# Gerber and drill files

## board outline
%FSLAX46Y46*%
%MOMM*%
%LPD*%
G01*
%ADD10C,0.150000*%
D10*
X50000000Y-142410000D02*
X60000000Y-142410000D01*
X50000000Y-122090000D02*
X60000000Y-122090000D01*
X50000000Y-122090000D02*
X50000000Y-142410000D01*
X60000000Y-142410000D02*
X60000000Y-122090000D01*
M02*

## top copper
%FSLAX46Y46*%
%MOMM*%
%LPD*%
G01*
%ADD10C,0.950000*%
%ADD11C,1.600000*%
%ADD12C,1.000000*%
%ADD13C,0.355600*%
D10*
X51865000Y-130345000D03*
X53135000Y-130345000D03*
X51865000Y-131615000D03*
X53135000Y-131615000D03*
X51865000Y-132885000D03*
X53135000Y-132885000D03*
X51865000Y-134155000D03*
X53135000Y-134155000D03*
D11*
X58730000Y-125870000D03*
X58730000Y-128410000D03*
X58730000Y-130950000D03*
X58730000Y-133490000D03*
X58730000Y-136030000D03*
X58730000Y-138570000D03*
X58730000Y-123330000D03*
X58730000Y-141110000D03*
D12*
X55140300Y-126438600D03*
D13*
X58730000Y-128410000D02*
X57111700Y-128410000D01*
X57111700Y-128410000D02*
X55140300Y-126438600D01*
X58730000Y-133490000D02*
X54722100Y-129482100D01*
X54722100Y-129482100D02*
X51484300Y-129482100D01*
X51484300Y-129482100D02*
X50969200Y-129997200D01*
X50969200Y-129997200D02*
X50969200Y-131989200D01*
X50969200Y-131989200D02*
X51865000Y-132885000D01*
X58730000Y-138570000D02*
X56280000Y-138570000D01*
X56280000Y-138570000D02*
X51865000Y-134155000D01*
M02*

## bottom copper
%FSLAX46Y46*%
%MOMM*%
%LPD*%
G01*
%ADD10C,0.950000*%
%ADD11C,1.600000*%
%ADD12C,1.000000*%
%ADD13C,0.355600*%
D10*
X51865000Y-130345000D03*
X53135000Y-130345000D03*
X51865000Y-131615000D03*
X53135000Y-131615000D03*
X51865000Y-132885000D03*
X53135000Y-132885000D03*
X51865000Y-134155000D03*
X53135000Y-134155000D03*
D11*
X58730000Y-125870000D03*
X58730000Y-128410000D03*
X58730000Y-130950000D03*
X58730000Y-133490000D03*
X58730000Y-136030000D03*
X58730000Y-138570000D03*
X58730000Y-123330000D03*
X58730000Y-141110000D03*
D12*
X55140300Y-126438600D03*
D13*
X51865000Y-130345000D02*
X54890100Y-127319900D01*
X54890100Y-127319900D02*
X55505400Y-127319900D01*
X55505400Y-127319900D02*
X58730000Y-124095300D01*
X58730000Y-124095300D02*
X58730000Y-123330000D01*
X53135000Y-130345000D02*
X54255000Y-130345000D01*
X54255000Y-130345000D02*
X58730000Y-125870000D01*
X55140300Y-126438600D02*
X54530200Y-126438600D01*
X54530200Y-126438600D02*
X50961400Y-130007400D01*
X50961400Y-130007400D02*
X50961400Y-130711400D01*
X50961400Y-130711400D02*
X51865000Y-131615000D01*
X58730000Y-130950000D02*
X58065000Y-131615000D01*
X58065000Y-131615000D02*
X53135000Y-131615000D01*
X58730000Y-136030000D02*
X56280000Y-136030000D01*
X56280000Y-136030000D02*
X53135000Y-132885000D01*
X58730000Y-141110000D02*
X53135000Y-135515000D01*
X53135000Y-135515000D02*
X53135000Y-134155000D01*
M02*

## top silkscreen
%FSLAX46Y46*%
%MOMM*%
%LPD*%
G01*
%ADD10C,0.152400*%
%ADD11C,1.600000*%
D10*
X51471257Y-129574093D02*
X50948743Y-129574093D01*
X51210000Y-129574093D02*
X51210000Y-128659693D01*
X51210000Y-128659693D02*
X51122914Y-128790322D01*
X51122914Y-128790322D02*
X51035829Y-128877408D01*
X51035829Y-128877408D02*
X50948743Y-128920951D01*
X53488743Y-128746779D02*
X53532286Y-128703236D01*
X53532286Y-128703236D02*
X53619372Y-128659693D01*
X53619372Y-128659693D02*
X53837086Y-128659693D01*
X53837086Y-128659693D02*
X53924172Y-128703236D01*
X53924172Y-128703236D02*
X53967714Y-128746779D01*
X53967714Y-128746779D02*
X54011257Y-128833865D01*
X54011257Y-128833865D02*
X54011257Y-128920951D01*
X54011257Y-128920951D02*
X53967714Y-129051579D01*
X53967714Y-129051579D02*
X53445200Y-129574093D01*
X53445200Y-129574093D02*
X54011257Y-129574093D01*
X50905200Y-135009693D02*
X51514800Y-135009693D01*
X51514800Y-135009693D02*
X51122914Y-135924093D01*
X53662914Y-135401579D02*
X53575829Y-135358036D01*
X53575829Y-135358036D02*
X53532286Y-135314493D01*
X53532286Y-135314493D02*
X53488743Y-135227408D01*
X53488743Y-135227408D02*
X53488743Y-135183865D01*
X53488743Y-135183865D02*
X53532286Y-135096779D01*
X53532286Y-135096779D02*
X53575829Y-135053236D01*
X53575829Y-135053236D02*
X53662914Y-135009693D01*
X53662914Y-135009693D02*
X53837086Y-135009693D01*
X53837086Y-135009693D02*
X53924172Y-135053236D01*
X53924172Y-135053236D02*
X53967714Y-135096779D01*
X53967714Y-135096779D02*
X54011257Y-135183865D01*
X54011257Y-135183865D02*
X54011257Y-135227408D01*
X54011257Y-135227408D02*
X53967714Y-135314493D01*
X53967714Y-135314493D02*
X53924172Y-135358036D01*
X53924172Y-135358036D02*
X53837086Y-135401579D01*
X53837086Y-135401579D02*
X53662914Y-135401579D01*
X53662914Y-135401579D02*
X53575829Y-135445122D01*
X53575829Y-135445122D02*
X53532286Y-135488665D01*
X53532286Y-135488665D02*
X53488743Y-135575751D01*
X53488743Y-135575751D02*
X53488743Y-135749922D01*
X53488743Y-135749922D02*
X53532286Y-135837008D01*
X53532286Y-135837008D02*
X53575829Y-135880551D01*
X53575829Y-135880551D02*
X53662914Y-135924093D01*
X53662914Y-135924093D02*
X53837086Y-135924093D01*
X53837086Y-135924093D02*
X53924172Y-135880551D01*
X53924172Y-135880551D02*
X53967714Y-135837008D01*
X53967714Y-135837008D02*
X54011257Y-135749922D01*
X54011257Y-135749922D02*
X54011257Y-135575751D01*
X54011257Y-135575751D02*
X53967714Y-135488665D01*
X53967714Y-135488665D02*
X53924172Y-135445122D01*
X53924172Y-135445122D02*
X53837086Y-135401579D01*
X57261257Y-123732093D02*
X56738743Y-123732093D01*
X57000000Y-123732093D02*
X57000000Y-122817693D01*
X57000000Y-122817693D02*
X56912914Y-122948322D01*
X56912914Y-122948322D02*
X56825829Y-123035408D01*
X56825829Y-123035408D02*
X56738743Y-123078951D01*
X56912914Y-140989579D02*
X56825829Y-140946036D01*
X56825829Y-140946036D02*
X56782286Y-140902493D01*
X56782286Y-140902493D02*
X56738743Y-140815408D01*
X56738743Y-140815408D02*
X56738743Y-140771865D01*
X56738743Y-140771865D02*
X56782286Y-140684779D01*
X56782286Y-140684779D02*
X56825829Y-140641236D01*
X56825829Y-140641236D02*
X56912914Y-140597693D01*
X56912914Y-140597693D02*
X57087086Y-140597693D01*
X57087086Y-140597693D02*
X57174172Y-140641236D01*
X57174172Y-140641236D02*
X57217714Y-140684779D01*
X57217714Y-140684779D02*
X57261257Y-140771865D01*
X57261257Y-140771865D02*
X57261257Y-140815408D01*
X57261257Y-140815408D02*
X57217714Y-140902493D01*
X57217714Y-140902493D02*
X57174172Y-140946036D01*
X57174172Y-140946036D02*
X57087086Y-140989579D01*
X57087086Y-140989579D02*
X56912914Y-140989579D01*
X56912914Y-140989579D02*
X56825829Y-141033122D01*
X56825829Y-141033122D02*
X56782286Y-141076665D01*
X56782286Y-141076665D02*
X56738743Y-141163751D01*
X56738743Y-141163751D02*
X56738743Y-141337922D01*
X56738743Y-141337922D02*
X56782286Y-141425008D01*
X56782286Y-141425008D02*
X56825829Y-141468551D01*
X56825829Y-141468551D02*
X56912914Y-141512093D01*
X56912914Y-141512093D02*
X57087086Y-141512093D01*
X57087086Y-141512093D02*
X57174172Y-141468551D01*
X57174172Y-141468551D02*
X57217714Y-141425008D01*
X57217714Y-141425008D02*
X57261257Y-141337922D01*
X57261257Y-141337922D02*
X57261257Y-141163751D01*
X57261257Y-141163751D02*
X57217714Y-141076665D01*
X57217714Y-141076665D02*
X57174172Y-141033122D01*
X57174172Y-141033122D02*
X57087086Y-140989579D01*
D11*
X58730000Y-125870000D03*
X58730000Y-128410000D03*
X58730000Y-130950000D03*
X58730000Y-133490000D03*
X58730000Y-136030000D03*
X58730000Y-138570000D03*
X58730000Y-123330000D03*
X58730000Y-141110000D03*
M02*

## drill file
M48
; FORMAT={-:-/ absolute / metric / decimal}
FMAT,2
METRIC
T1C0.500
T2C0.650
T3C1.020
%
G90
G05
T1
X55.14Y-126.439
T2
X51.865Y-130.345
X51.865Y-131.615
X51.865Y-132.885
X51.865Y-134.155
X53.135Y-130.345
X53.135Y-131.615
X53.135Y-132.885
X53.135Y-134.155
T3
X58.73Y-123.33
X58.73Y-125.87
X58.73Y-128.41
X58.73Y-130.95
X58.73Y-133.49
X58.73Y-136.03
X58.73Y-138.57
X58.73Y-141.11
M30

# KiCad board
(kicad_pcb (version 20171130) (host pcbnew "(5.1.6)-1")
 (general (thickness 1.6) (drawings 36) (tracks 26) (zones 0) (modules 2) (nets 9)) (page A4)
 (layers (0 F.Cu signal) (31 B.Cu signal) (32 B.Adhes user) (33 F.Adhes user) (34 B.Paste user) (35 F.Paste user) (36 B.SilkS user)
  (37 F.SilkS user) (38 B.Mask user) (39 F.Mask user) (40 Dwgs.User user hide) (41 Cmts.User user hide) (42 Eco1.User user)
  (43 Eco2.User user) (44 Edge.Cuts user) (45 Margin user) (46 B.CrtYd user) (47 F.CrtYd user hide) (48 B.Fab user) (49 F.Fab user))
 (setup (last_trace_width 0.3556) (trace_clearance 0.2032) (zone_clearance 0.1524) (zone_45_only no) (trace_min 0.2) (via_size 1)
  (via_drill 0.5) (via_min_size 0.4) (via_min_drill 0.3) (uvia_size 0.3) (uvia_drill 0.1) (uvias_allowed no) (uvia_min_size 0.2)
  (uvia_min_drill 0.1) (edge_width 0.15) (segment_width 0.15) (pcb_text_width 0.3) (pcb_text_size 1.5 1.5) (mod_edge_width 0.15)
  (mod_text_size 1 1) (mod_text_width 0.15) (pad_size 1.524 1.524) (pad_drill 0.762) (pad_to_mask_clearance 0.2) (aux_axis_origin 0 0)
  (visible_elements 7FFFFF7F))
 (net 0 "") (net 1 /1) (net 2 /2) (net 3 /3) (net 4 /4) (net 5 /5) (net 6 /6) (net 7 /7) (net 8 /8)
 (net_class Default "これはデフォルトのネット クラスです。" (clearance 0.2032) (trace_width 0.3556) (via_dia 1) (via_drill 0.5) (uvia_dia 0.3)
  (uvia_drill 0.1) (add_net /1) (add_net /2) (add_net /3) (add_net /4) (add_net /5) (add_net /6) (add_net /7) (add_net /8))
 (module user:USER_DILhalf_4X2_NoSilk (layer F.Cu) (at 52.5 132.25)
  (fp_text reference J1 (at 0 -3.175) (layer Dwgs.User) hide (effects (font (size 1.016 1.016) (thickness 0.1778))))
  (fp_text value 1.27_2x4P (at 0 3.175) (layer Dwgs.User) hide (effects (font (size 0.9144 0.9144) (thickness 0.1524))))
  (pad 1 thru_hole circle (at -0.635 -1.905) (size 0.95 0.95) (drill 0.65) (layers *.Cu *.Mask) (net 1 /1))
  (pad 2 thru_hole circle (at 0.635 -1.905) (size 0.95 0.95) (drill 0.65) (layers *.Cu *.Mask) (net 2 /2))
  (pad 3 thru_hole circle (at -0.635 -0.635) (size 0.95 0.95) (drill 0.65) (layers *.Cu *.Mask) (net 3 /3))
  (pad 4 thru_hole circle (at 0.635 -0.635) (size 0.95 0.95) (drill 0.65) (layers *.Cu *.Mask) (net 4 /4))
  (pad 5 thru_hole circle (at -0.635 0.635) (size 0.95 0.95) (drill 0.65) (layers *.Cu *.Mask) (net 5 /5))
  (pad 6 thru_hole circle (at 0.635 0.635) (size 0.95 0.95) (drill 0.65) (layers *.Cu *.Mask) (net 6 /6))
  (pad 7 thru_hole circle (at -0.635 1.905) (size 0.95 0.95) (drill 0.65) (layers *.Cu *.Mask) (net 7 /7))
  (pad 8 thru_hole circle (at 0.635 1.905) (size 0.95 0.95) (drill 0.65) (layers *.Cu *.Mask) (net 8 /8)))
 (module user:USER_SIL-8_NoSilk (layer F.Cu) (at 58.73 132.22 270)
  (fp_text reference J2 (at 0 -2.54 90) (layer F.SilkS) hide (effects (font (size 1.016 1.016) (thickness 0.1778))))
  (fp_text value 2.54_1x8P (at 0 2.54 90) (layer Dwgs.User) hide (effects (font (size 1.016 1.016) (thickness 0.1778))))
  (pad 2 thru_hole circle (at -6.35 0 270) (size 1.6 1.6) (drill 1.02) (layers *.Cu *.Mask F.SilkS) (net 2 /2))
  (pad 3 thru_hole circle (at -3.81 0 270) (size 1.6 1.6) (drill 1.02) (layers *.Cu *.Mask F.SilkS) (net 3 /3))
  (pad 4 thru_hole circle (at -1.27 0 270) (size 1.6 1.6) (drill 1.02) (layers *.Cu *.Mask F.SilkS) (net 4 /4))
  (pad 5 thru_hole circle (at 1.27 0 270) (size 1.6 1.6) (drill 1.02) (layers *.Cu *.Mask F.SilkS) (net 5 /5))
  (pad 6 thru_hole circle (at 3.81 0 270) (size 1.6 1.6) (drill 1.02) (layers *.Cu *.Mask F.SilkS) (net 6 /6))
  (pad 7 thru_hole circle (at 6.35 0 270) (size 1.6 1.6) (drill 1.02) (layers *.Cu *.Mask F.SilkS) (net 7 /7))
  (pad 1 thru_hole circle (at -8.89 0 270) (size 1.6 1.6) (drill 1.02) (layers *.Cu *.Mask F.SilkS) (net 1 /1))
  (pad 8 thru_hole circle (at 8.89 0 270) (size 1.6 1.6) (drill 1.02) (layers *.Cu *.Mask F.SilkS) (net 8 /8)))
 (gr_line (start 50 142.41) (end 60 142.41) (angle 90) (layer Edge.Cuts) (width 0.15))
 (gr_line (start 50 122.09) (end 60 122.09) (angle 90) (layer Edge.Cuts) (width 0.15))
 (gr_line (start 50 122.09) (end 50 142.41) (angle 90) (layer Edge.Cuts) (width 0.15))
 (gr_line (start 60 142.41) (end 60 122.09) (angle 90) (layer Edge.Cuts) (width 0.15))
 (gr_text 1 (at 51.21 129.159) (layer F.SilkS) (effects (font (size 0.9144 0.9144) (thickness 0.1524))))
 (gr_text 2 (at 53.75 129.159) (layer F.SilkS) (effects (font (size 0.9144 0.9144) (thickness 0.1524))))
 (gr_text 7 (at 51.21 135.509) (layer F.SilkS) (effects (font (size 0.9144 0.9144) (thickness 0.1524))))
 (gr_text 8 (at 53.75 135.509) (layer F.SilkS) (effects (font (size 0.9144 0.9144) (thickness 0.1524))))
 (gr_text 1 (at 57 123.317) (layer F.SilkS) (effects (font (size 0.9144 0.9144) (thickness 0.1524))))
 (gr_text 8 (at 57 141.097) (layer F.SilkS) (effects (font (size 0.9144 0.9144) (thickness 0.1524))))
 (segment (start 51.865 130.345) (end 54.8901 127.3199) (width 0.3556) (layer B.Cu) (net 1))
 (segment (start 54.8901 127.3199) (end 55.5054 127.3199) (width 0.3556) (layer B.Cu) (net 1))
 (segment (start 55.5054 127.3199) (end 58.73 124.0953) (width 0.3556) (layer B.Cu) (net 1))
 (segment (start 58.73 124.0953) (end 58.73 123.33) (width 0.3556) (layer B.Cu) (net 1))
 (segment (start 53.135 130.345) (end 54.255 130.345) (width 0.3556) (layer B.Cu) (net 2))
 (segment (start 54.255 130.345) (end 58.73 125.87) (width 0.3556) (layer B.Cu) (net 2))
 (segment (start 55.1403 126.4386) (end 54.5302 126.4386) (width 0.3556) (layer B.Cu) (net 3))
 (segment (start 54.5302 126.4386) (end 50.9614 130.0074) (width 0.3556) (layer B.Cu) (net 3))
 (segment (start 50.9614 130.0074) (end 50.9614 130.7114) (width 0.3556) (layer B.Cu) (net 3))
 (segment (start 50.9614 130.7114) (end 51.865 131.615) (width 0.3556) (layer B.Cu) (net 3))
 (segment (start 58.73 128.41) (end 57.1117 128.41) (width 0.3556) (layer F.Cu) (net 3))
 (segment (start 57.1117 128.41) (end 55.1403 126.4386) (width 0.3556) (layer F.Cu) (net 3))
 (via (at 55.1403 126.4386) (size 1) (layers F.Cu B.Cu) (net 3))
 (segment (start 58.73 130.95) (end 58.065 131.615) (width 0.3556) (layer B.Cu) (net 4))
 (segment (start 58.065 131.615) (end 53.135 131.615) (width 0.3556) (layer B.Cu) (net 4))
 (segment (start 58.73 133.49) (end 54.7221 129.4821) (width 0.3556) (layer F.Cu) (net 5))
 (segment (start 54.7221 129.4821) (end 51.4843 129.4821) (width 0.3556) (layer F.Cu) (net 5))
 (segment (start 51.4843 129.4821) (end 50.9692 129.9972) (width 0.3556) (layer F.Cu) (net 5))
 (segment (start 50.9692 129.9972) (end 50.9692 131.9892) (width 0.3556) (layer F.Cu) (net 5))
 (segment (start 50.9692 131.9892) (end 51.865 132.885) (width 0.3556) (layer F.Cu) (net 5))
 (segment (start 58.73 136.03) (end 56.28 136.03) (width 0.3556) (layer B.Cu) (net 6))
 (segment (start 56.28 136.03) (end 53.135 132.885) (width 0.3556) (layer B.Cu) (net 6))
 (segment (start 58.73 138.57) (end 56.28 138.57) (width 0.3556) (layer F.Cu) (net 7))
 (segment (start 56.28 138.57) (end 51.865 134.155) (width 0.3556) (layer F.Cu) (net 7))
 (segment (start 58.73 141.11) (end 53.135 135.515) (width 0.3556) (layer B.Cu) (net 8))
 (segment (start 53.135 135.515) (end 53.135 134.155) (width 0.3556) (layer B.Cu) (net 8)))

